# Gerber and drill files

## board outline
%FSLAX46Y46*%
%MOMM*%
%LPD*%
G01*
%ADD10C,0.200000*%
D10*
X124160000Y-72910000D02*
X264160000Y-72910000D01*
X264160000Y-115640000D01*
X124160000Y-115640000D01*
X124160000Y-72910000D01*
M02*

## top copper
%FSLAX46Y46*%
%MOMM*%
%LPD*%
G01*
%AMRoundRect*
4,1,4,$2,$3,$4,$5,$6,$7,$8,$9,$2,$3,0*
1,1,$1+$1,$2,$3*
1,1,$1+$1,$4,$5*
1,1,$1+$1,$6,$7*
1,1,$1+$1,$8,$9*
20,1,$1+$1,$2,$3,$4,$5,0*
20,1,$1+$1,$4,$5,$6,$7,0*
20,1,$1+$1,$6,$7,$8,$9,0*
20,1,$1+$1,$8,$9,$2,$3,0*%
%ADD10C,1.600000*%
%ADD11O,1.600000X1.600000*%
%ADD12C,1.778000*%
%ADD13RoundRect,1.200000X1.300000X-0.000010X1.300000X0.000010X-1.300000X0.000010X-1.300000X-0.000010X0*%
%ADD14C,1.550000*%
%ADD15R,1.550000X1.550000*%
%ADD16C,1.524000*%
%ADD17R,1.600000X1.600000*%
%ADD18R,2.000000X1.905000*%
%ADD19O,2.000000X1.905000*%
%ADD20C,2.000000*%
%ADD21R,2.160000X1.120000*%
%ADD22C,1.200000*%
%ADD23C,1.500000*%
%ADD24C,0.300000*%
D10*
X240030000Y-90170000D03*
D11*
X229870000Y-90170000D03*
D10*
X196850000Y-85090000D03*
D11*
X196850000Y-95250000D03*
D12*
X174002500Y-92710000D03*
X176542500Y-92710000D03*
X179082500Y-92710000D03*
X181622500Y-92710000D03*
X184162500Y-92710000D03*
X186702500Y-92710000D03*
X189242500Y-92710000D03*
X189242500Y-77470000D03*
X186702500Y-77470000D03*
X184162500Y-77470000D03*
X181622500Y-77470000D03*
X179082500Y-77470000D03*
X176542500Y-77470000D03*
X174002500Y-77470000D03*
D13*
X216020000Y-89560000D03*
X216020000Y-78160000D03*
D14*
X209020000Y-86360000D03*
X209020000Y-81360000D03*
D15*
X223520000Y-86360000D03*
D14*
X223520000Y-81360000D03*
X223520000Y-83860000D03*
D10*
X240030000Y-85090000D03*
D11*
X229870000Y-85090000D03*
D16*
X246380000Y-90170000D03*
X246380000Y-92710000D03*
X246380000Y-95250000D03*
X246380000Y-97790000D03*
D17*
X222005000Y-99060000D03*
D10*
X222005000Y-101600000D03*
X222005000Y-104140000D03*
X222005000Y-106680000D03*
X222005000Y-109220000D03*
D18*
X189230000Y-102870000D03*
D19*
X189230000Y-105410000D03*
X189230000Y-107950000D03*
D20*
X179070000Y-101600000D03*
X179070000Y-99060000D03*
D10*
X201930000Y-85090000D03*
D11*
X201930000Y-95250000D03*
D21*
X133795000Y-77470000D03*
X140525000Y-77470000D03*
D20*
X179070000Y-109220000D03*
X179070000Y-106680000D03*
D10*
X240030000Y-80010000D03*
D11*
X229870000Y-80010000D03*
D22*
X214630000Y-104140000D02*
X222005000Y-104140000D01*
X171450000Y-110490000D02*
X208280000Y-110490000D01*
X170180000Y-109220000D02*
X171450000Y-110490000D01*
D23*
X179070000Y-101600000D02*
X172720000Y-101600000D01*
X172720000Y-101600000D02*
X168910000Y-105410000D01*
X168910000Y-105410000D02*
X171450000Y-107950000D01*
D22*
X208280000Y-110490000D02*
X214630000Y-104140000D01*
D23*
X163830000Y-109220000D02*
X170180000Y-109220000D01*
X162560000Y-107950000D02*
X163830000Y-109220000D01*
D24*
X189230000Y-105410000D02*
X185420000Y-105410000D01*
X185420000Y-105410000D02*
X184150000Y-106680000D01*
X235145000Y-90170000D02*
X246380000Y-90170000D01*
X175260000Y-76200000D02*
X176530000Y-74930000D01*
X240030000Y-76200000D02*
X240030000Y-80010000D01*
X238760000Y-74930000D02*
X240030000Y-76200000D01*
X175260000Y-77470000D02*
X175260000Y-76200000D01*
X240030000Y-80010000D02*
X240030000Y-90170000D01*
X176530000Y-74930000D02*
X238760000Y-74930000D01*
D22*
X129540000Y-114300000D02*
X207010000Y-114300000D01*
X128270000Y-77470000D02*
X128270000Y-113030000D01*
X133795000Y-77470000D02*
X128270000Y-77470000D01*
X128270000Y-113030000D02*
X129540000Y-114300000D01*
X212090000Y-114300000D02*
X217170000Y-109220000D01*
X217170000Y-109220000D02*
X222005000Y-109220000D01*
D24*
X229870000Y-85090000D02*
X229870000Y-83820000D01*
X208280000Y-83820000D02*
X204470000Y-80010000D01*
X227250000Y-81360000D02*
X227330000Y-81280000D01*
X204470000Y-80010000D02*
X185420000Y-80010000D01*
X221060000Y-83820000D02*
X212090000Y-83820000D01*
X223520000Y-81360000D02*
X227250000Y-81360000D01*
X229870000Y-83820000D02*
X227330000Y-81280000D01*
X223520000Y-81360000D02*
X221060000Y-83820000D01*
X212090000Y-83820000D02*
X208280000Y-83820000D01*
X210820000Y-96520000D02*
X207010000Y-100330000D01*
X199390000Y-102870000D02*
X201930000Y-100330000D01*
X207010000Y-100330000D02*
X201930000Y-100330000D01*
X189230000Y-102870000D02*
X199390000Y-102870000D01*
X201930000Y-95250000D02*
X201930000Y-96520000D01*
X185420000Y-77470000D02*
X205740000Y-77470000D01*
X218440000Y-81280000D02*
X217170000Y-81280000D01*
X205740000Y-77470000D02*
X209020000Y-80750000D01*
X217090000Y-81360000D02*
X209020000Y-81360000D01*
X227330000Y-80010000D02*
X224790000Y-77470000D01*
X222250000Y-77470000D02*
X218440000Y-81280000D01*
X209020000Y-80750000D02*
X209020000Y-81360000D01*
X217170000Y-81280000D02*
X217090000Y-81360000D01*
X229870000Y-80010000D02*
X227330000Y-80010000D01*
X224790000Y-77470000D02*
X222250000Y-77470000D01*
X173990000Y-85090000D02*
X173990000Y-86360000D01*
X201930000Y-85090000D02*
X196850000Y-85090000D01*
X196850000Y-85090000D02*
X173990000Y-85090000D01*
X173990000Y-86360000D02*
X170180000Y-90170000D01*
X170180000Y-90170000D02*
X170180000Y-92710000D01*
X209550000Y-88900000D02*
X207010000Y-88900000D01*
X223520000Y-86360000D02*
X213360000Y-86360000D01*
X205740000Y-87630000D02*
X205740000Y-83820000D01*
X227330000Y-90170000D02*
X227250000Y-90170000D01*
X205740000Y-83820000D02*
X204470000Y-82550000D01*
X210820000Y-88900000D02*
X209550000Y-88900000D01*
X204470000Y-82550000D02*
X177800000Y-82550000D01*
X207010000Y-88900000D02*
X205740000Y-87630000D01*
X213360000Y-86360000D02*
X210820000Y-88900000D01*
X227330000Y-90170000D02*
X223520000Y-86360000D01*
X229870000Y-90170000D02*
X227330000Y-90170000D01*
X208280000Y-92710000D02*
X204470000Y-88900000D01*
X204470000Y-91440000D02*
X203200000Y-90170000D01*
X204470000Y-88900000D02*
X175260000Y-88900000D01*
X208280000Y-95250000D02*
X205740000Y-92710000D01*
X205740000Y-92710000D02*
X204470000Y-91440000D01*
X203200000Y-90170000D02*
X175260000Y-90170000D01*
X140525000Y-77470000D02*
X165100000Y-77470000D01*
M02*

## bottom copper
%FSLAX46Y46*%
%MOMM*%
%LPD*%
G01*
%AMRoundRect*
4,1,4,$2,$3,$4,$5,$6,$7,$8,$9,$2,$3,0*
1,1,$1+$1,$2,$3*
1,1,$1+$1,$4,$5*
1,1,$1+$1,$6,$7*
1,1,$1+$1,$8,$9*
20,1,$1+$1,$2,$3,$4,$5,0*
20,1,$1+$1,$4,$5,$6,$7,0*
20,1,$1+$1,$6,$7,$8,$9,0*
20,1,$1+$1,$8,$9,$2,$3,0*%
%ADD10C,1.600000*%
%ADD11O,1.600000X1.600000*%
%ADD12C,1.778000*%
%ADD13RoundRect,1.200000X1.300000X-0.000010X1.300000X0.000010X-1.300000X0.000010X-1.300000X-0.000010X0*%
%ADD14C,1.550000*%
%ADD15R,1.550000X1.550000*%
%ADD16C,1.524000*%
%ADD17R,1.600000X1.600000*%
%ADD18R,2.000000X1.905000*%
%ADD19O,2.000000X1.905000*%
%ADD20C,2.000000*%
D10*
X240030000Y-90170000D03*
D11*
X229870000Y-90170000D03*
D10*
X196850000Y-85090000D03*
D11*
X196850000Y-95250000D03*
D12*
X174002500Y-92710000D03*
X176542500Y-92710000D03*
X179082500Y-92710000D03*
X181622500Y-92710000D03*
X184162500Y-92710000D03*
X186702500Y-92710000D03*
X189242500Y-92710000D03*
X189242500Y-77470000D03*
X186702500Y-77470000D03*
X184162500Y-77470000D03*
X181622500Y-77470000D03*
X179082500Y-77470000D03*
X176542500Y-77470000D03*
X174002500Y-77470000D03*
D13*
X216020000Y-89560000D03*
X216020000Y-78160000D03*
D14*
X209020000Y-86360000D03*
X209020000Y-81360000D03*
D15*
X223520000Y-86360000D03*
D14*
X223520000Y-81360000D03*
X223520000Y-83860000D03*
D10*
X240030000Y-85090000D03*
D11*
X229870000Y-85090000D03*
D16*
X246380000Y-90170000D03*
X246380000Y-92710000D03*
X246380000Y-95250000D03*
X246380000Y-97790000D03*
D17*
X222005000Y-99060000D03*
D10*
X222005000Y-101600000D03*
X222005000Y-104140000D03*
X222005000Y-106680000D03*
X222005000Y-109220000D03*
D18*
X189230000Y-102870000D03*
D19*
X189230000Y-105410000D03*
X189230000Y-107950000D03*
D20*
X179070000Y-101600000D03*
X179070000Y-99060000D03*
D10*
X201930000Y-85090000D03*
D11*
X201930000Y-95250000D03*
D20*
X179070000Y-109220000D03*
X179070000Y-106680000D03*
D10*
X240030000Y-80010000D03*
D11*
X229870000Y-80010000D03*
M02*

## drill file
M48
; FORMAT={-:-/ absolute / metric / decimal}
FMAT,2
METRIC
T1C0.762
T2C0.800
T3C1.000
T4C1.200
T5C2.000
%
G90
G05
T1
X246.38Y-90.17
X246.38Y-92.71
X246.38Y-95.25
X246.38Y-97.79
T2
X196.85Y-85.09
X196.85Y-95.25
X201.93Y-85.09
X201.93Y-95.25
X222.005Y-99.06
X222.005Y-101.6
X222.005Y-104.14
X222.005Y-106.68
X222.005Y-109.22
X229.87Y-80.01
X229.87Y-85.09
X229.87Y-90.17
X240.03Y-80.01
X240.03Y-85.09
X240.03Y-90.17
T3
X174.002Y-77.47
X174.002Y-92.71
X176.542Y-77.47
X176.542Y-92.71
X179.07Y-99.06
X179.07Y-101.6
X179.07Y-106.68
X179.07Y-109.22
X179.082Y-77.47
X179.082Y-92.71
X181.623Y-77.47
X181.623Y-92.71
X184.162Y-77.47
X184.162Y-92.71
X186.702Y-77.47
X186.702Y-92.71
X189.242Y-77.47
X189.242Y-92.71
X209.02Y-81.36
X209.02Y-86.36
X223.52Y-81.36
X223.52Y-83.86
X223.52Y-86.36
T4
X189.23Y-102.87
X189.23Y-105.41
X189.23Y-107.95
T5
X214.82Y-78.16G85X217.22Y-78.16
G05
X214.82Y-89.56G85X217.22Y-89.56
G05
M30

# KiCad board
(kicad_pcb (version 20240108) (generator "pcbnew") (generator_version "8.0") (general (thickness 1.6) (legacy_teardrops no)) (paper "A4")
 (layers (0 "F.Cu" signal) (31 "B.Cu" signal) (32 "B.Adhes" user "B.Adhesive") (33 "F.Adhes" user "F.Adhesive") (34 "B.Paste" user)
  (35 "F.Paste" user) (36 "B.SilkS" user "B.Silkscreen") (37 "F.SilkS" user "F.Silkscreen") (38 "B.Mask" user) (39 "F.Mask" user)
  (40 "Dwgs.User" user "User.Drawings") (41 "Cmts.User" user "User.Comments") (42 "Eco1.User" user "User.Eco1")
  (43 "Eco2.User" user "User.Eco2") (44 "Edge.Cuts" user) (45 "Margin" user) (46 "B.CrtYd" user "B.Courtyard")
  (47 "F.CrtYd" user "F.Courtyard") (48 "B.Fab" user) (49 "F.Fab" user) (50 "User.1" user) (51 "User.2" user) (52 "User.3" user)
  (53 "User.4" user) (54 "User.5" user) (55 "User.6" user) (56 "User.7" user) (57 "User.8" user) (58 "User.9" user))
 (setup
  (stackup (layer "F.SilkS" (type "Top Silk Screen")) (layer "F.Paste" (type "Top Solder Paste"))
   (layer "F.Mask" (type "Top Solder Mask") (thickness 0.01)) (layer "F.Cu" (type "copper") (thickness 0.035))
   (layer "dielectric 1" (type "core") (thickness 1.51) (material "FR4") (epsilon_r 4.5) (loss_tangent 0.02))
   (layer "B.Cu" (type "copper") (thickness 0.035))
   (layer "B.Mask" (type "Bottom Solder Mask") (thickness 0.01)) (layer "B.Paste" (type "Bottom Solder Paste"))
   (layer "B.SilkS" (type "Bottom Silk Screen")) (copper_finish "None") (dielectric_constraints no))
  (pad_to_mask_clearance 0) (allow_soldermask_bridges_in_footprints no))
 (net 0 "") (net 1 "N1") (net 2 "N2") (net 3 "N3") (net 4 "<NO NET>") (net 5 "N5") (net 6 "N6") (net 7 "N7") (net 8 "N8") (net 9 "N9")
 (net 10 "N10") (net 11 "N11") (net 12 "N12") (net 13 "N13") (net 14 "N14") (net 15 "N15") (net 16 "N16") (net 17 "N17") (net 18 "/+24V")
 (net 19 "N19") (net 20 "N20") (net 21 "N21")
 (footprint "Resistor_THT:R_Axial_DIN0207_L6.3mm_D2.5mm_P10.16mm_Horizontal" (layer "F.Cu") (at 240.03 90.17 180)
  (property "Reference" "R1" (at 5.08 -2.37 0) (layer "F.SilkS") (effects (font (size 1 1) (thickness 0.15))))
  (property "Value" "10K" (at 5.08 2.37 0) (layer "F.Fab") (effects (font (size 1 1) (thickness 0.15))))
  (pad "1" thru_hole circle (at 0 0 180) (size 1.6 1.6) (drill 0.8) (layers "*.Cu" "*.Mask") (remove_unused_layers no) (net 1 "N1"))
  (pad "2" thru_hole oval (at 10.16 0 180) (size 1.6 1.6) (drill 0.8) (layers "*.Cu" "*.Mask") (remove_unused_layers no) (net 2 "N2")))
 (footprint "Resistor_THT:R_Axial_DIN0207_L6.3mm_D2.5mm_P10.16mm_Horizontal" (layer "F.Cu") (at 196.85 85.09 -90)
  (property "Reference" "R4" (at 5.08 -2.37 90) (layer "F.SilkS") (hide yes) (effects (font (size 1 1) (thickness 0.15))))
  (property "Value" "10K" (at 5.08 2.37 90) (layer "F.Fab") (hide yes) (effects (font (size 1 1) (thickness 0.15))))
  (pad "1" thru_hole circle (at 0 0 270) (size 1.6 1.6) (drill 0.8) (layers "*.Cu" "*.Mask") (remove_unused_layers no) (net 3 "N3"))
  (pad "2" thru_hole oval (at 10.16 0 270) (size 1.6 1.6) (drill 0.8) (layers "*.Cu" "*.Mask") (remove_unused_layers no) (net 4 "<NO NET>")))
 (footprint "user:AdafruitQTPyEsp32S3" (layer "F.Cu") (at 174.0025 92.71 90)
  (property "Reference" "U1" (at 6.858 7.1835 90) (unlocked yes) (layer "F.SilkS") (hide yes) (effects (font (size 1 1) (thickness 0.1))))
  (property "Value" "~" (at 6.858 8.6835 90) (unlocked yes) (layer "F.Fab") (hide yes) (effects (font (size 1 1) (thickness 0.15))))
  (pad "1" thru_hole circle (at 0 0 90) (size 1.778 1.778) (drill 1) (layers "*.Cu" "*.Mask") (remove_unused_layers no) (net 3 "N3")
   (solder_mask_margin 0.0508) (thermal_bridge_angle 0))
  (pad "2" thru_hole circle (at 0 2.54 90) (size 1.778 1.778) (drill 1) (layers "*.Cu" "*.Mask") (remove_unused_layers no) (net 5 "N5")
   (solder_mask_margin 0.0508) (thermal_bridge_angle 0))
  (pad "3" thru_hole circle (at 0 5.08 90) (size 1.778 1.778) (drill 1) (layers "*.Cu" "*.Mask") (remove_unused_layers no) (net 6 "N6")
   (solder_mask_margin 0.0508) (thermal_bridge_angle 0))
  (pad "4" thru_hole circle (at 0 7.62 90) (size 1.778 1.778) (drill 1) (layers "*.Cu" "*.Mask") (remove_unused_layers no) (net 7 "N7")
   (solder_mask_margin 0.0508) (thermal_bridge_angle 0))
  (pad "5" thru_hole circle (at 0 10.16 90) (size 1.778 1.778) (drill 1) (layers "*.Cu" "*.Mask") (remove_unused_layers no) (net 2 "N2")
   (solder_mask_margin 0.0508) (thermal_bridge_angle 0))
  (pad "6" thru_hole circle (at 0 12.7 90) (size 1.778 1.778) (drill 1) (layers "*.Cu" "*.Mask") (remove_unused_layers no) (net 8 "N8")
   (solder_mask_margin 0.0508) (thermal_bridge_angle 0))
  (pad "7" thru_hole circle (at 0 15.24 90) (size 1.778 1.778) (drill 1) (layers "*.Cu" "*.Mask") (remove_unused_layers no) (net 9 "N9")
   (solder_mask_margin 0.0508) (thermal_bridge_angle 0))
  (pad "8" thru_hole circle (at 15.24 15.24 270) (size 1.778 1.778) (drill 1) (layers "*.Cu" "*.Mask") (remove_unused_layers no)
   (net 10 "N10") (solder_mask_margin 0.0508) (thermal_bridge_angle 0))
  (pad "9" thru_hole circle (at 15.24 12.7 270) (size 1.778 1.778) (drill 1) (layers "*.Cu" "*.Mask") (remove_unused_layers no)
   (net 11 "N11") (solder_mask_margin 0.0508) (thermal_bridge_angle 0))
  (pad "10" thru_hole circle (at 15.24 10.16 270) (size 1.778 1.778) (drill 1) (layers "*.Cu" "*.Mask") (remove_unused_layers no)
   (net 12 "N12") (solder_mask_margin 0.0508) (thermal_bridge_angle 0))
  (pad "11" thru_hole circle (at 15.24 7.62 270) (size 1.778 1.778) (drill 1) (layers "*.Cu" "*.Mask") (remove_unused_layers no)
   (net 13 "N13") (solder_mask_margin 0.0508) (thermal_bridge_angle 0))
  (pad "12" thru_hole circle (at 15.24 5.08 270) (size 1.778 1.778) (drill 1) (layers "*.Cu" "*.Mask") (remove_unused_layers no)
   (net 1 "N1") (solder_mask_margin 0.0508) (thermal_bridge_angle 0))
  (pad "13" thru_hole circle (at 15.24 2.54 270) (size 1.778 1.778) (drill 1) (layers "*.Cu" "*.Mask") (remove_unused_layers no)
   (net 4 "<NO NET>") (solder_mask_margin 0.0508) (thermal_bridge_angle 0))
  (pad "14" thru_hole circle (at 15.24 0 270) (size 1.778 1.778) (drill 1) (layers "*.Cu" "*.Mask") (remove_unused_layers no) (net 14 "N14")
   (solder_mask_margin 0.0508) (thermal_bridge_angle 0)))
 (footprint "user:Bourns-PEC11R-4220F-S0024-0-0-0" (layer "F.Cu") (at 216.02 83.86 90)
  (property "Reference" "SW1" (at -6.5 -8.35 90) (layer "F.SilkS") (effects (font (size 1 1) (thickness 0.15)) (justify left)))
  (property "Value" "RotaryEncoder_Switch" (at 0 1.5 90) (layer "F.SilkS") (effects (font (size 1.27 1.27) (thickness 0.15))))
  (pad "" thru_hole roundrect (at -5.7 0 90) (size 2.4 5) (drill oval 2 4.4) (layers "*.Cu" "*.Mask") (remove_unused_layers no)
   (roundrect_rratio 0.5))
  (pad "" thru_hole roundrect (at 5.7 0 90) (size 2.4 5) (drill oval 2 4.4) (layers "*.Cu" "*.Mask") (remove_unused_layers no)
   (roundrect_rratio 0.5))
  (pad "1" thru_hole circle (at -2.5 -7 90) (size 1.55 1.55) (drill 1) (layers "*.Cu" "*.Mask") (remove_unused_layers no) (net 4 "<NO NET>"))
  (pad "2" thru_hole circle (at 2.5 -7 90) (size 1.55 1.55) (drill 1) (layers "*.Cu" "*.Mask") (remove_unused_layers no) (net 10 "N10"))
  (pad "A" thru_hole rect (at -2.5 7.5 90) (size 1.55 1.55) (drill 1) (layers "*.Cu" "*.Mask") (remove_unused_layers no) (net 2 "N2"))
  (pad "B" thru_hole circle (at 2.5 7.5 90) (size 1.55 1.55) (drill 1) (layers "*.Cu" "*.Mask") (remove_unused_layers no) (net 6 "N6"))
  (pad "C" thru_hole circle (at 0 7.5 90) (size 1.55 1.55) (drill 1) (layers "*.Cu" "*.Mask") (remove_unused_layers no) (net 4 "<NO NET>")))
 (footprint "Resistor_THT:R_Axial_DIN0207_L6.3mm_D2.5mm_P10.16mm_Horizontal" (layer "F.Cu") (at 240.03 85.09 180)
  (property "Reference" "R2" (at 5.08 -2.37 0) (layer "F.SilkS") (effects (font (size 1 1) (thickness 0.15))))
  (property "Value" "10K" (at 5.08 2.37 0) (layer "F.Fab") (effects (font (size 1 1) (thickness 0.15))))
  (pad "1" thru_hole circle (at 0 0 180) (size 1.6 1.6) (drill 0.8) (layers "*.Cu" "*.Mask") (remove_unused_layers no) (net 1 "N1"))
  (pad "2" thru_hole oval (at 10.16 0 180) (size 1.6 1.6) (drill 0.8) (layers "*.Cu" "*.Mask") (remove_unused_layers no) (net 6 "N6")))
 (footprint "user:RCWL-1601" (layer "F.Cu") (at 246.38 90.17 -90)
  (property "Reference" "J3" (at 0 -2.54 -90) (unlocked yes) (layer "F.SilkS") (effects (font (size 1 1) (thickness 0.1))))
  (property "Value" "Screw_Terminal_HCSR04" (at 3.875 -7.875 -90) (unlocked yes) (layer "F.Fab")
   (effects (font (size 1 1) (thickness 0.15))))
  (pad "1" thru_hole circle (at 0 0 270) (size 1.524 1.524) (drill 0.762) (layers "*.Cu" "*.Mask") (remove_unused_layers no) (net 1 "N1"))
  (pad "2" thru_hole circle (at 2.54 0 270) (size 1.524 1.524) (drill 0.762) (layers "*.Cu" "*.Mask") (remove_unused_layers no)
   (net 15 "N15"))
  (pad "3" thru_hole circle (at 5.08 0 270) (size 1.524 1.524) (drill 0.762) (layers "*.Cu" "*.Mask") (remove_unused_layers no) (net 9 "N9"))
  (pad "4" thru_hole circle (at 7.62 0 270) (size 1.524 1.524) (drill 0.762) (layers "*.Cu" "*.Mask") (remove_unused_layers no)
   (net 4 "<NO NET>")))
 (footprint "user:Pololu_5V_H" (layer "F.Cu") (at 222.005 104.14 -90)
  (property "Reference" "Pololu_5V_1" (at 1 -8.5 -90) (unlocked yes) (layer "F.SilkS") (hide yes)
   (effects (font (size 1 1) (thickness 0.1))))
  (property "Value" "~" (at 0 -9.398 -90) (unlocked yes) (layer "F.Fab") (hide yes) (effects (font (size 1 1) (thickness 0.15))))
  (pad "1" thru_hole rect (at -5.08 0 270) (size 1.6 1.6) (drill 0.8) (layers "*.Cu" "*.Mask") (remove_unused_layers no) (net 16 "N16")
   (thermal_bridge_angle 45))
  (pad "2" thru_hole circle (at -2.54 0 270) (size 1.6 1.6) (drill 0.8) (layers "*.Cu" "*.Mask") (remove_unused_layers no) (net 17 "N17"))
  (pad "3" thru_hole circle (at 0 0 270) (size 1.6 1.6) (drill 0.8) (layers "*.Cu" "*.Mask") (remove_unused_layers no) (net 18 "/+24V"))
  (pad "4" thru_hole circle (at 2.54 0 270) (size 1.6 1.6) (drill 0.8) (layers "*.Cu" "*.Mask") (remove_unused_layers no) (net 4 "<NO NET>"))
  (pad "5" thru_hole circle (at 5.08 0 270) (size 1.6 1.6) (drill 0.8) (layers "*.Cu" "*.Mask") (remove_unused_layers no) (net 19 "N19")))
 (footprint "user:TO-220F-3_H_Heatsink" (layer "F.Cu") (at 189.23 102.87 -90)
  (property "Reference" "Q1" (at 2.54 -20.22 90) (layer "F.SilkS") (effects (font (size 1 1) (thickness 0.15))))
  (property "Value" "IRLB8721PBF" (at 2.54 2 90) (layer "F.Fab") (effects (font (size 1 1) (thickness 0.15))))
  (pad "1" thru_hole rect (at 0 0 270) (size 1.905 2) (drill 1.2) (layers "*.Cu" "*.Mask") (remove_unused_layers no) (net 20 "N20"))
  (pad "2" thru_hole oval (at 2.54 0 270) (size 1.905 2) (drill 1.2) (layers "*.Cu" "*.Mask") (remove_unused_layers no) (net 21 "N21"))
  (pad "3" thru_hole oval (at 5.08 0 270) (size 1.905 2) (drill 1.2) (layers "*.Cu" "*.Mask") (remove_unused_layers no) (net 4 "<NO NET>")))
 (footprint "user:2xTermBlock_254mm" (layer "F.Cu") (at 179.07 101.6 90)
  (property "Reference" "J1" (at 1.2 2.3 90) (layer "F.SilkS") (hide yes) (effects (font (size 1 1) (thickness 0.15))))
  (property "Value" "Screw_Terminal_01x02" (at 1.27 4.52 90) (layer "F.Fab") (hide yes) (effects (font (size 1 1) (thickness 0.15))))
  (pad "1" thru_hole circle (at 0 0 90) (size 2 2) (drill 1) (layers "*.Cu" "*.Mask") (remove_unused_layers no) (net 18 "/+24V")
   (thermal_bridge_angle 90))
  (pad "2" thru_hole circle (at 2.54 0 90) (size 2 2) (drill 1) (layers "*.Cu" "*.Mask") (remove_unused_layers no) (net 4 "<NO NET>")))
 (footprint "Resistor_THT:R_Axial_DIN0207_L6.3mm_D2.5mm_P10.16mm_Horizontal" (layer "F.Cu") (at 201.93 85.09 -90)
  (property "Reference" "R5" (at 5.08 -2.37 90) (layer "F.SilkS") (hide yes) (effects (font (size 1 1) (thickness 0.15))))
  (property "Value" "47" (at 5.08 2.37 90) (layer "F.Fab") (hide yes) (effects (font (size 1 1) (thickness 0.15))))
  (pad "1" thru_hole circle (at 0 0 270) (size 1.6 1.6) (drill 0.8) (layers "*.Cu" "*.Mask") (remove_unused_layers no) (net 3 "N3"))
  (pad "2" thru_hole oval (at 10.16 0 270) (size 1.6 1.6) (drill 0.8) (layers "*.Cu" "*.Mask") (remove_unused_layers no) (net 20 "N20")))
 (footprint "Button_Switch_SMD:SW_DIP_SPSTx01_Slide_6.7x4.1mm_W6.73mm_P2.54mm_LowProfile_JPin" (layer "F.Cu") (at 137.16 77.47)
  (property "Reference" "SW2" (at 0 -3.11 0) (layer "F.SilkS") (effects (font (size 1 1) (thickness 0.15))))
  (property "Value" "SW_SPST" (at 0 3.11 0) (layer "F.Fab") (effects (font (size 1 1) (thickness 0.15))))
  (pad "1" smd rect (at -3.365 0) (size 2.16 1.12) (layers "F.Cu" "F.Paste" "F.Mask") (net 19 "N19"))
  (pad "2" smd rect (at 3.365 0) (size 2.16 1.12) (layers "F.Cu" "F.Paste" "F.Mask") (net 14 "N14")))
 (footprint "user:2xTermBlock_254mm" (layer "F.Cu") (at 179.07 109.22 90)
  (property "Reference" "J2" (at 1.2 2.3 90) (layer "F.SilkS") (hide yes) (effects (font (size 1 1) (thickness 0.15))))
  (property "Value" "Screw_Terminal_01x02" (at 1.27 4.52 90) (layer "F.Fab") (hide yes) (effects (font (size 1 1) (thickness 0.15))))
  (pad "1" thru_hole circle (at 0 0 90) (size 2 2) (drill 1) (layers "*.Cu" "*.Mask") (remove_unused_layers no) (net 18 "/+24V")
   (thermal_bridge_angle 90))
  (pad "2" thru_hole circle (at 2.54 0 90) (size 2 2) (drill 1) (layers "*.Cu" "*.Mask") (remove_unused_layers no) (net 21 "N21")))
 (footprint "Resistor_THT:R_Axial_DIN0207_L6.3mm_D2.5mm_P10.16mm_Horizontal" (layer "F.Cu") (at 240.03 80.01 180)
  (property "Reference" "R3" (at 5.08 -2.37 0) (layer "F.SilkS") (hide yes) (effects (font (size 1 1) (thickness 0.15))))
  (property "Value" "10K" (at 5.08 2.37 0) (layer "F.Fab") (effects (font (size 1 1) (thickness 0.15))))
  (pad "1" thru_hole circle (at 0 0 180) (size 1.6 1.6) (drill 0.8) (layers "*.Cu" "*.Mask") (remove_unused_layers no) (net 1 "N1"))
  (pad "2" thru_hole oval (at 10.16 0 180) (size 1.6 1.6) (drill 0.8) (layers "*.Cu" "*.Mask") (remove_unused_layers no) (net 10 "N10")))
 (gr_rect (start 124.16 72.91) (end 264.16 115.64) (stroke (width 0.2) (type default)) (fill none) (layer "Edge.Cuts"))
 (segment (start 214.63 104.14) (end 222.005 104.14) (width 1.2) (layer "F.Cu") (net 18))
 (segment (start 171.45 110.49) (end 208.28 110.49) (width 1.2) (layer "F.Cu") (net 18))
 (segment (start 170.18 109.22) (end 171.45 110.49) (width 1.2) (layer "F.Cu") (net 18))
 (segment (start 179.07 101.6) (end 172.72 101.6) (width 1.5) (layer "F.Cu") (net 18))
 (segment (start 172.72 101.6) (end 168.91 105.41) (width 1.5) (layer "F.Cu") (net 18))
 (segment (start 168.91 105.41) (end 171.45 107.95) (width 1.5) (layer "F.Cu") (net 18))
 (segment (start 208.28 110.49) (end 214.63 104.14) (width 1.2) (layer "F.Cu") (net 18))
 (segment (start 163.83 109.22) (end 170.18 109.22) (width 1.5) (layer "F.Cu") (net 18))
 (segment (start 162.56 107.95) (end 163.83 109.22) (width 1.5) (layer "F.Cu") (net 18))
 (segment (start 189.23 105.41) (end 185.42 105.41) (width 0.3) (layer "F.Cu") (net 21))
 (segment (start 185.42 105.41) (end 184.15 106.68) (width 0.3) (layer "F.Cu") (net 21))
 (segment (start 235.145 90.17) (end 246.38 90.17) (width 0.3) (layer "F.Cu") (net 1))
 (segment (start 175.26 76.2) (end 176.53 74.93) (width 0.3) (layer "F.Cu") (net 1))
 (segment (start 240.03 76.2) (end 240.03 80.01) (width 0.3) (layer "F.Cu") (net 1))
 (segment (start 238.76 74.93) (end 240.03 76.2) (width 0.3) (layer "F.Cu") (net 1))
 (segment (start 175.26 77.47) (end 175.26 76.2) (width 0.3) (layer "F.Cu") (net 1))
 (segment (start 240.03 80.01) (end 240.03 90.17) (width 0.3) (layer "F.Cu") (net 1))
 (segment (start 176.53 74.93) (end 238.76 74.93) (width 0.3) (layer "F.Cu") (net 1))
 (segment (start 129.54 114.3) (end 207.01 114.3) (width 1.2) (layer "F.Cu") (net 19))
 (segment (start 128.27 77.47) (end 128.27 113.03) (width 1.2) (layer "F.Cu") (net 19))
 (segment (start 133.795 77.47) (end 128.27 77.47) (width 1.2) (layer "F.Cu") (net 19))
 (segment (start 128.27 113.03) (end 129.54 114.3) (width 1.2) (layer "F.Cu") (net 19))
 (segment (start 212.09 114.3) (end 217.17 109.22) (width 1.2) (layer "F.Cu") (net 19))
 (segment (start 217.17 109.22) (end 222.005 109.22) (width 1.2) (layer "F.Cu") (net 19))
 (segment (start 229.87 85.09) (end 229.87 83.82) (width 0.3) (layer "F.Cu") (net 6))
 (segment (start 208.28 83.82) (end 204.47 80.01) (width 0.3) (layer "F.Cu") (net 6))
 (segment (start 227.25 81.36) (end 227.33 81.28) (width 0.3) (layer "F.Cu") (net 6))
 (segment (start 204.47 80.01) (end 185.42 80.01) (width 0.3) (layer "F.Cu") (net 6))
 (segment (start 221.06 83.82) (end 212.09 83.82) (width 0.3) (layer "F.Cu") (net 6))
 (segment (start 223.52 81.36) (end 227.25 81.36) (width 0.3) (layer "F.Cu") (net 6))
 (segment (start 229.87 83.82) (end 227.33 81.28) (width 0.3) (layer "F.Cu") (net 6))
 (segment (start 223.52 81.36) (end 221.06 83.82) (width 0.3) (layer "F.Cu") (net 6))
 (segment (start 212.09 83.82) (end 208.28 83.82) (width 0.3) (layer "F.Cu") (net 6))
 (segment (start 210.82 96.52) (end 207.01 100.33) (width 0.3) (layer "F.Cu") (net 20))
 (segment (start 199.39 102.87) (end 201.93 100.33) (width 0.3) (layer "F.Cu") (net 20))
 (segment (start 207.01 100.33) (end 201.93 100.33) (width 0.3) (layer "F.Cu") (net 20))
 (segment (start 189.23 102.87) (end 199.39 102.87) (width 0.3) (layer "F.Cu") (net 20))
 (segment (start 201.93 95.25) (end 201.93 96.52) (width 0.3) (layer "F.Cu") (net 20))
 (segment (start 185.42 77.47) (end 205.74 77.47) (width 0.3) (layer "F.Cu") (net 10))
 (segment (start 218.44 81.28) (end 217.17 81.28) (width 0.3) (layer "F.Cu") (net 10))
 (segment (start 205.74 77.47) (end 209.02 80.75) (width 0.3) (layer "F.Cu") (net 10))
 (segment (start 217.09 81.36) (end 209.02 81.36) (width 0.3) (layer "F.Cu") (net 10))
 (segment (start 227.33 80.01) (end 224.79 77.47) (width 0.3) (layer "F.Cu") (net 10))
 (segment (start 222.25 77.47) (end 218.44 81.28) (width 0.3) (layer "F.Cu") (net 10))
 (segment (start 209.02 80.75) (end 209.02 81.36) (width 0.3) (layer "F.Cu") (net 10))
 (segment (start 217.17 81.28) (end 217.09 81.36) (width 0.3) (layer "F.Cu") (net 10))
 (segment (start 229.87 80.01) (end 227.33 80.01) (width 0.3) (layer "F.Cu") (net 10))
 (segment (start 224.79 77.47) (end 222.25 77.47) (width 0.3) (layer "F.Cu") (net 10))
 (segment (start 173.99 85.09) (end 173.99 86.36) (width 0.3) (layer "F.Cu") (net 3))
 (segment (start 201.93 85.09) (end 196.85 85.09) (width 0.3) (layer "F.Cu") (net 3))
 (segment (start 196.85 85.09) (end 173.99 85.09) (width 0.3) (layer "F.Cu") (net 3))
 (segment (start 173.99 86.36) (end 170.18 90.17) (width 0.3) (layer "F.Cu") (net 3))
 (segment (start 170.18 90.17) (end 170.18 92.71) (width 0.3) (layer "F.Cu") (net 3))
 (segment (start 209.55 88.9) (end 207.01 88.9) (width 0.3) (layer "F.Cu") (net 2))
 (segment (start 223.52 86.36) (end 213.36 86.36) (width 0.3) (layer "F.Cu") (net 2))
 (segment (start 205.74 87.63) (end 205.74 83.82) (width 0.3) (layer "F.Cu") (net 2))
 (segment (start 227.33 90.17) (end 227.25 90.17) (width 0.3) (layer "F.Cu") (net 2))
 (segment (start 205.74 83.82) (end 204.47 82.55) (width 0.3) (layer "F.Cu") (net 2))
 (segment (start 210.82 88.9) (end 209.55 88.9) (width 0.3) (layer "F.Cu") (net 2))
 (segment (start 204.47 82.55) (end 177.8 82.55) (width 0.3) (layer "F.Cu") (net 2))
 (segment (start 207.01 88.9) (end 205.74 87.63) (width 0.3) (layer "F.Cu") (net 2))
 (segment (start 213.36 86.36) (end 210.82 88.9) (width 0.3) (layer "F.Cu") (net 2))
 (segment (start 227.33 90.17) (end 223.52 86.36) (width 0.3) (layer "F.Cu") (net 2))
 (segment (start 229.87 90.17) (end 227.33 90.17) (width 0.3) (layer "F.Cu") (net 2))
 (segment (start 208.28 92.71) (end 204.47 88.9) (width 0.3) (layer "F.Cu") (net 15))
 (segment (start 204.47 91.44) (end 203.2 90.17) (width 0.3) (layer "F.Cu") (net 15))
 (segment (start 204.47 88.9) (end 175.26 88.9) (width 0.3) (layer "F.Cu") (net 15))
 (segment (start 208.28 95.25) (end 205.74 92.71) (width 0.3) (layer "F.Cu") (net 15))
 (segment (start 205.74 92.71) (end 204.47 91.44) (width 0.3) (layer "F.Cu") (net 15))
 (segment (start 203.2 90.17) (end 175.26 90.17) (width 0.3) (layer "F.Cu") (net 15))
 (segment (start 140.525 77.47) (end 165.1 77.47) (width 0.3) (layer "F.Cu") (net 14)))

